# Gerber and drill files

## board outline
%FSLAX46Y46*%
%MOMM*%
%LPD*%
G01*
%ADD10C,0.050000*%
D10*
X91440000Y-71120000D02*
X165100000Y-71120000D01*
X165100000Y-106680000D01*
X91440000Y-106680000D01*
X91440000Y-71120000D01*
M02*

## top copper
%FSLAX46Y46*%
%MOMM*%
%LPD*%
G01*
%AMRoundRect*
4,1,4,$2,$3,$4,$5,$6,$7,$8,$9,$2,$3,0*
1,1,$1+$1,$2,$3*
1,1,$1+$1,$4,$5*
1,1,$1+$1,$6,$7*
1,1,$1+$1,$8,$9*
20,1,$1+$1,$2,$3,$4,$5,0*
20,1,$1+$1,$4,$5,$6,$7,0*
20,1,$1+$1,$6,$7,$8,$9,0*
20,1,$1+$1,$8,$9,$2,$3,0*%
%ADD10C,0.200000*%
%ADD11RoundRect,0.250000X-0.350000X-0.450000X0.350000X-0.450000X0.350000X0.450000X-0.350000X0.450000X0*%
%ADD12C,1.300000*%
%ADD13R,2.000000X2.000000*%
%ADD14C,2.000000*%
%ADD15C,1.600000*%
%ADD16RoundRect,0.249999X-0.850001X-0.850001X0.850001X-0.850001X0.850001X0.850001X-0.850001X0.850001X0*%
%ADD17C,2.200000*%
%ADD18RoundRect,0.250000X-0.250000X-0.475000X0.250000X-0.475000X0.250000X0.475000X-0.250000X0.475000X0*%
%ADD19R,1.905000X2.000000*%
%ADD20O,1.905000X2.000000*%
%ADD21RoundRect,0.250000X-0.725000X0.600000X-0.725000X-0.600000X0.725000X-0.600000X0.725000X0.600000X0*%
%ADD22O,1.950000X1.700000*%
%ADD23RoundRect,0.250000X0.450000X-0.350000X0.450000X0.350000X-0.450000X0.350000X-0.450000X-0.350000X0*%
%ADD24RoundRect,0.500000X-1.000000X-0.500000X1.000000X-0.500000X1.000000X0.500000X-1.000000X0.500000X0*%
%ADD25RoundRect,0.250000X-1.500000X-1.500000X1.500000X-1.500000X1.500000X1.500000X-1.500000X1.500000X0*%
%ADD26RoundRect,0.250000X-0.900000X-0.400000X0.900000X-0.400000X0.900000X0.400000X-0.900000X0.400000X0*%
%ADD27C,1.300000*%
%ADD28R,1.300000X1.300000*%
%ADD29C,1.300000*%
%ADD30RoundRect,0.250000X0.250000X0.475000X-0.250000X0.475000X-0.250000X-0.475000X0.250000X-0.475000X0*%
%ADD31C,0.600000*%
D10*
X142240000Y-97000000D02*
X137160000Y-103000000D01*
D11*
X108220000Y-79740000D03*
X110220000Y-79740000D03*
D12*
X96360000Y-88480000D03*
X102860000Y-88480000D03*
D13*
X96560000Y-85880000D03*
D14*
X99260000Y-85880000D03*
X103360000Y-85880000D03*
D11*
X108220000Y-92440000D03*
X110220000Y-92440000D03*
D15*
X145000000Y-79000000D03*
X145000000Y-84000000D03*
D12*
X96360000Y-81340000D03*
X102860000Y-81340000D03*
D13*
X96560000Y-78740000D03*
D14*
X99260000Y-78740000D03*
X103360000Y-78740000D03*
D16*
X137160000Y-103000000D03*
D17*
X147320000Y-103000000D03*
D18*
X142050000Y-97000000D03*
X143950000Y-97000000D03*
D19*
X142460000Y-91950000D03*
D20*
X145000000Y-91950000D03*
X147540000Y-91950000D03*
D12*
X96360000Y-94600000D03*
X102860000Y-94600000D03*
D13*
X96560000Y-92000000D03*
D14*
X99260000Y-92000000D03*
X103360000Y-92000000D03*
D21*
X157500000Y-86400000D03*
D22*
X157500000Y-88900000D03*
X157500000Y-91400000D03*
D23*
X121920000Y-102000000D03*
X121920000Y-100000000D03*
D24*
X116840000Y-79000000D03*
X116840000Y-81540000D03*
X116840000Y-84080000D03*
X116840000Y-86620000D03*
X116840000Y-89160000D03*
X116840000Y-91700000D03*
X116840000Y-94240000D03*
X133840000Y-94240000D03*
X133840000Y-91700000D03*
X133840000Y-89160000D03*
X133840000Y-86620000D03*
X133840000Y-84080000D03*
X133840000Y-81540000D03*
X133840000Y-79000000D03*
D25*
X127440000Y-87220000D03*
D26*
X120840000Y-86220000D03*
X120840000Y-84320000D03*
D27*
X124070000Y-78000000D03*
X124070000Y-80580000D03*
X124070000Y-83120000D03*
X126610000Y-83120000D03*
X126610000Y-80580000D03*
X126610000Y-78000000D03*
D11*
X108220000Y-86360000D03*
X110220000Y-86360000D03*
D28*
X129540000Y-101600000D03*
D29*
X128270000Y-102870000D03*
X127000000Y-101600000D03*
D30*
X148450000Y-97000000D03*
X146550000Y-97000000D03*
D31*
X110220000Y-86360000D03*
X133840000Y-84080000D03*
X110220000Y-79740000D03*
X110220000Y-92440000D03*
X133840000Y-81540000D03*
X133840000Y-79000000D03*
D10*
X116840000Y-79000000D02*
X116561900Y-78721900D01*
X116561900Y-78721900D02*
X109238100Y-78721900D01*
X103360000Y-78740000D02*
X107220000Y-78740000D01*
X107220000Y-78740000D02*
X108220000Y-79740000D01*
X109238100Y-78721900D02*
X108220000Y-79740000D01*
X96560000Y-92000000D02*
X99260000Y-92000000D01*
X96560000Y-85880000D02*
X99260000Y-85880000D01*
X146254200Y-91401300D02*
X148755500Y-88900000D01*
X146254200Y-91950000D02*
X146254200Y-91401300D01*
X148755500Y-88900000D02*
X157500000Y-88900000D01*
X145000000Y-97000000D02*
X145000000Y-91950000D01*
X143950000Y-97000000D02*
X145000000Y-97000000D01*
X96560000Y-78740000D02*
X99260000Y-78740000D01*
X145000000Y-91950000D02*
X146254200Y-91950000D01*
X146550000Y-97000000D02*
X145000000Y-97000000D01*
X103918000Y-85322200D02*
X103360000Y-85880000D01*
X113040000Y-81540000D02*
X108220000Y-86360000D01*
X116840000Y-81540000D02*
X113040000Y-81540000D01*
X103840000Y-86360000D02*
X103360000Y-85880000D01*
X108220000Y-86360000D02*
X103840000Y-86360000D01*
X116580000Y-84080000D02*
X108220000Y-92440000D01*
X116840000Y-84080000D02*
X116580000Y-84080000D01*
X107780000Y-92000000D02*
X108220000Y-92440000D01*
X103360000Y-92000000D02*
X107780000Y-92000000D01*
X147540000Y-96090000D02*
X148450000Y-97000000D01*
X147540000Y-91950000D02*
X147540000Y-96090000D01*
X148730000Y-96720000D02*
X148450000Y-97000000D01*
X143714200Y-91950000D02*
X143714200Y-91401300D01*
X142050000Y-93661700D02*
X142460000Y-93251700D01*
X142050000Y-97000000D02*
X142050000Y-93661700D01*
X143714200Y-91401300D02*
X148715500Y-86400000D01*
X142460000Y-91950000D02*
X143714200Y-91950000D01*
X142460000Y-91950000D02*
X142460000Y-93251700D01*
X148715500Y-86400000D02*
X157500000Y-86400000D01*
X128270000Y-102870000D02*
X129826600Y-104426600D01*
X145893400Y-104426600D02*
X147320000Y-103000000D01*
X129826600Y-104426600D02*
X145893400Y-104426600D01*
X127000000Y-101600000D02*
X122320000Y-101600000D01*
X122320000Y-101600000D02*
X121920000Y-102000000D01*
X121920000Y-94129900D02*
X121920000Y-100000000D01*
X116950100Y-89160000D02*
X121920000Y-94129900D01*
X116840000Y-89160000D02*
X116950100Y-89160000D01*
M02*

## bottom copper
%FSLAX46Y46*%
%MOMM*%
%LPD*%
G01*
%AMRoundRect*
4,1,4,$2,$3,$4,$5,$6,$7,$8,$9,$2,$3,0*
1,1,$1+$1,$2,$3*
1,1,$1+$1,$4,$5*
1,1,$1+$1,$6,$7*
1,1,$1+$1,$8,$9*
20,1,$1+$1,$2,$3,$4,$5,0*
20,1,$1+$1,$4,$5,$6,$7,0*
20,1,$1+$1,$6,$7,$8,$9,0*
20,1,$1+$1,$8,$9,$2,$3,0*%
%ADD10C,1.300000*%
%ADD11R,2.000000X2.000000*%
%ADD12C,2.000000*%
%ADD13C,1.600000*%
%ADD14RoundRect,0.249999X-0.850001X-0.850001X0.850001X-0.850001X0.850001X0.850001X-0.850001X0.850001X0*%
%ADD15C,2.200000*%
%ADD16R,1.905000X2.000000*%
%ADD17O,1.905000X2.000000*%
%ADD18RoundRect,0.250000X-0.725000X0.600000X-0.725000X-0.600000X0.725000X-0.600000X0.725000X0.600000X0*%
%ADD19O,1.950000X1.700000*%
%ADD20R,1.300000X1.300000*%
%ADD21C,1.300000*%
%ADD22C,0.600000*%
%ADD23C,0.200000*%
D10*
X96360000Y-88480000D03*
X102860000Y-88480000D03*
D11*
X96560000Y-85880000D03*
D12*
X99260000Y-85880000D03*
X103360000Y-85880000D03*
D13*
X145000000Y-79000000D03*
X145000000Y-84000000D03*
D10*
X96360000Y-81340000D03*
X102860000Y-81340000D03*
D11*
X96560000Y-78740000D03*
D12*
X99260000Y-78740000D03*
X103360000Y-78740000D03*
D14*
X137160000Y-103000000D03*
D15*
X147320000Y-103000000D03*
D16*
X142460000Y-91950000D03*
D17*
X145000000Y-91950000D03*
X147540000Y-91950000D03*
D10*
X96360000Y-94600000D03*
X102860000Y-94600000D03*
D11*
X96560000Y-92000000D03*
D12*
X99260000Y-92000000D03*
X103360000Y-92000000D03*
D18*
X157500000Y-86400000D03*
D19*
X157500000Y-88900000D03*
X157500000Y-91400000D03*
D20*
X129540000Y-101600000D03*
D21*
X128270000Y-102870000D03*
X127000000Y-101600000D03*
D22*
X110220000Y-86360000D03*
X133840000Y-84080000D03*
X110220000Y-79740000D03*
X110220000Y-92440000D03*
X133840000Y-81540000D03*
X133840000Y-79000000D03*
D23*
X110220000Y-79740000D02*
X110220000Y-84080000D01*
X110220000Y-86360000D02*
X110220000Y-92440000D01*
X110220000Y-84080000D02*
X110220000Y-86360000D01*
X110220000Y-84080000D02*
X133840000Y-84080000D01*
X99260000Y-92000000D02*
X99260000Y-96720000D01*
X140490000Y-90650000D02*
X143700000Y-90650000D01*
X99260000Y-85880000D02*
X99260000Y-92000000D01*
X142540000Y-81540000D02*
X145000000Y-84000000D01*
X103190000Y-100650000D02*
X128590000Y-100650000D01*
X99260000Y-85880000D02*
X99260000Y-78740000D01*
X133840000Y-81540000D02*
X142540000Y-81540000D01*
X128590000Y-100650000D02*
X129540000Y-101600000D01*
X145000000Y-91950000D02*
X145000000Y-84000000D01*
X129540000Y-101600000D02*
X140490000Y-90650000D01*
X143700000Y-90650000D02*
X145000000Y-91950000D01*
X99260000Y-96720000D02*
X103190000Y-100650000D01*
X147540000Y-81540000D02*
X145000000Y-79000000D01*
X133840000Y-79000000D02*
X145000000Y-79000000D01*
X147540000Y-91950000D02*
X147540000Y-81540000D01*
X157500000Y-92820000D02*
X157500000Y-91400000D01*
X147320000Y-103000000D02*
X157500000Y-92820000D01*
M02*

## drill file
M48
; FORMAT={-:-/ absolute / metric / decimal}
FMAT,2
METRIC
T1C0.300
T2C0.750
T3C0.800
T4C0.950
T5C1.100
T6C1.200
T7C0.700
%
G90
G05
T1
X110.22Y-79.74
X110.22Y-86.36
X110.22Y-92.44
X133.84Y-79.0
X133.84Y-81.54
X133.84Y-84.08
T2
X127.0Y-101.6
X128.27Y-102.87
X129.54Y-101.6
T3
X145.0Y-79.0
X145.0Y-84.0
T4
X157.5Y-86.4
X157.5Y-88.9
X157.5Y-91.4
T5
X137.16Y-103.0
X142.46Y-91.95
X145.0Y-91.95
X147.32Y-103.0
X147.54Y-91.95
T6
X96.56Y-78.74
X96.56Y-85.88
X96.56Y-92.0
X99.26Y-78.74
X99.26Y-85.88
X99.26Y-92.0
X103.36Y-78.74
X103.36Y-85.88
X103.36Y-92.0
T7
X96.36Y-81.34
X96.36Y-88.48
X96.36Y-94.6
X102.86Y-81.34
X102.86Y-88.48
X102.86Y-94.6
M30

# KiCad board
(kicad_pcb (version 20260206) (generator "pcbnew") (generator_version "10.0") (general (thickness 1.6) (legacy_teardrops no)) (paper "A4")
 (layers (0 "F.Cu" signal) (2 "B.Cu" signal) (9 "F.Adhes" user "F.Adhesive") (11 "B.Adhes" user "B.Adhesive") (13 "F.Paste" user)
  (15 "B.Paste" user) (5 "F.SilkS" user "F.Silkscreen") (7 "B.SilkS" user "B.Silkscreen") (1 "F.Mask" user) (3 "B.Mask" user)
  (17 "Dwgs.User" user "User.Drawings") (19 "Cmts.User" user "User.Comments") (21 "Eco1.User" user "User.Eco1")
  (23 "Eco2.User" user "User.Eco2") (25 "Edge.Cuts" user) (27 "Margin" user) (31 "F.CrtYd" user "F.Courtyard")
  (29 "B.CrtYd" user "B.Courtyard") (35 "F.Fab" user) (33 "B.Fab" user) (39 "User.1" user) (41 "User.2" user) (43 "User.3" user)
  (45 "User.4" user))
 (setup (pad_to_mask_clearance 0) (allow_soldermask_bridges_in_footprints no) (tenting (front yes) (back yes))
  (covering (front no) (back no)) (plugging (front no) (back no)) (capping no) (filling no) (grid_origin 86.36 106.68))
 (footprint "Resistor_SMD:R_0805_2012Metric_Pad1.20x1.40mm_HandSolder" (layer "F.Cu") (at 109.22 79.74)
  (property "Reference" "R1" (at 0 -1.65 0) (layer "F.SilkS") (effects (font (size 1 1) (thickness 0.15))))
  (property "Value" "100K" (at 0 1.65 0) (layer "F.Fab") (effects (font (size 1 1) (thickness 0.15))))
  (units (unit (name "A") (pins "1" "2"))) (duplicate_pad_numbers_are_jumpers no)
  (pad "1" smd roundrect (at -1 0) (size 1.2 1.4) (layers "F.Cu" "F.Mask" "F.Paste") (roundrect_rratio 0.208333)
   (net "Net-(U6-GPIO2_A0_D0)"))
  (pad "2" smd roundrect (at 1 0) (size 1.2 1.4) (layers "F.Cu" "F.Mask" "F.Paste") (roundrect_rratio 0.208333) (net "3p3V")))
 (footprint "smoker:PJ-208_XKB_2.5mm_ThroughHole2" (layer "F.Cu") (at 94.86 85.88)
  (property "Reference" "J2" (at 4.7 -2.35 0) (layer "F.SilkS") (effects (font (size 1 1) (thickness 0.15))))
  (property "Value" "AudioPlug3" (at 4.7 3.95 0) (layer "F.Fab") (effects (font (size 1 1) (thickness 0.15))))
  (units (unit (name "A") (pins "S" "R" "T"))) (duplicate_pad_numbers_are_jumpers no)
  (pad "" np_thru_hole circle (at 1.5 2.6) (size 1.3 1.3) (drill 0.7) (layers "*.Cu" "*.Mask"))
  (pad "" np_thru_hole circle (at 8 2.6) (size 1.3 1.3) (drill 0.7) (layers "*.Cu" "*.Mask"))
  (pad "R" thru_hole rect (at 1.7 0) (size 2 2) (drill 1.2) (layers "*.Cu" "*.Mask") (remove_unused_layers no) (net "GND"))
  (pad "S" thru_hole circle (at 4.4 0) (size 2 2) (drill 1.2) (layers "*.Cu" "*.Mask") (remove_unused_layers no) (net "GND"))
  (pad "T" thru_hole circle (at 8.5 0) (size 2 2) (drill 1.2) (layers "*.Cu" "*.Mask") (remove_unused_layers no)
   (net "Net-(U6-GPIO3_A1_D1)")))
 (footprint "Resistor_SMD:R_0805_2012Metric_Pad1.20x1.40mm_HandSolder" (layer "F.Cu") (at 109.22 92.44)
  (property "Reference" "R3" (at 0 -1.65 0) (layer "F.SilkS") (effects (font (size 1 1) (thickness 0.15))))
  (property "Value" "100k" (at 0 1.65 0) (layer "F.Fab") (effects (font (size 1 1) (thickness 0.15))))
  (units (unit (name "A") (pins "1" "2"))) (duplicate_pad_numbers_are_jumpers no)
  (pad "1" smd roundrect (at -1 0) (size 1.2 1.4) (layers "F.Cu" "F.Mask" "F.Paste") (roundrect_rratio 0.208333)
   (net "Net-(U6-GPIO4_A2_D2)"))
  (pad "2" smd roundrect (at 1 0) (size 1.2 1.4) (layers "F.Cu" "F.Mask" "F.Paste") (roundrect_rratio 0.208333) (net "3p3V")))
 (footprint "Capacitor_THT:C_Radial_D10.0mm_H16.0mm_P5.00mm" (layer "F.Cu") (at 145 79 -90)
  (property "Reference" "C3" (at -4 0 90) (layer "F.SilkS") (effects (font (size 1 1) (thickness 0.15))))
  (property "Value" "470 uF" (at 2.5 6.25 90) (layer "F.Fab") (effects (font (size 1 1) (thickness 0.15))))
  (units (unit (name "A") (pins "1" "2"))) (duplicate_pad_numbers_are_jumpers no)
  (pad "1" thru_hole circle (at 0 0 270) (size 1.6 1.6) (drill 0.8) (layers "*.Cu" "*.Mask") (remove_unused_layers no) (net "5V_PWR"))
  (pad "2" thru_hole circle (at 5 0 270) (size 1.6 1.6) (drill 0.8) (layers "*.Cu" "*.Mask") (remove_unused_layers no) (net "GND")))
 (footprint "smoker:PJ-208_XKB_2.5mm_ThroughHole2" (layer "F.Cu") (at 94.86 78.74)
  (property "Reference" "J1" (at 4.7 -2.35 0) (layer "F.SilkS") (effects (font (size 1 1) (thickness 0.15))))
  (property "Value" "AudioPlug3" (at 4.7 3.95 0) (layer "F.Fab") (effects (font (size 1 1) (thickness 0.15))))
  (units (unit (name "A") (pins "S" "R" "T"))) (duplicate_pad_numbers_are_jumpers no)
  (pad "" np_thru_hole circle (at 1.5 2.6) (size 1.3 1.3) (drill 0.7) (layers "*.Cu" "*.Mask"))
  (pad "" np_thru_hole circle (at 8 2.6) (size 1.3 1.3) (drill 0.7) (layers "*.Cu" "*.Mask"))
  (pad "R" thru_hole rect (at 1.7 0) (size 2 2) (drill 1.2) (layers "*.Cu" "*.Mask") (remove_unused_layers no) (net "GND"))
  (pad "S" thru_hole circle (at 4.4 0) (size 2 2) (drill 1.2) (layers "*.Cu" "*.Mask") (remove_unused_layers no) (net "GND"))
  (pad "T" thru_hole circle (at 8.5 0) (size 2 2) (drill 1.2) (layers "*.Cu" "*.Mask") (remove_unused_layers no)
   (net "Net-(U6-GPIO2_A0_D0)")))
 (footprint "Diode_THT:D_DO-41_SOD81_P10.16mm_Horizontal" (layer "F.Cu") (at 137.16 103)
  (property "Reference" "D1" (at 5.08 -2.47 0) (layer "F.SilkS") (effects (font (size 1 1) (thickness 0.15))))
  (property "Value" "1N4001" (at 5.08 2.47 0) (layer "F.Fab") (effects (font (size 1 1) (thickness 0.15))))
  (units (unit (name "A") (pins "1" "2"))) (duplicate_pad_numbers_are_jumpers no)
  (pad "1" thru_hole roundrect (at 0 0) (size 2.2 2.2) (drill 1.1) (layers "*.Cu" "*.Mask") (remove_unused_layers no)
   (roundrect_rratio 0.113636) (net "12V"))
  (pad "2" thru_hole circle (at 10.16 0) (size 2.2 2.2) (drill 1.1) (layers "*.Cu" "*.Mask") (remove_unused_layers no) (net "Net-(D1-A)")))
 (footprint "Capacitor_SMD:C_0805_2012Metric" (layer "F.Cu") (at 143 97)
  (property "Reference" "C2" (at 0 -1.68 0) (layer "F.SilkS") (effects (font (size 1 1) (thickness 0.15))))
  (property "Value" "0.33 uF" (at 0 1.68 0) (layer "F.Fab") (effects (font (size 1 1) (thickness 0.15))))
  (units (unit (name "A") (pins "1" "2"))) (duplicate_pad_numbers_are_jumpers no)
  (pad "1" smd roundrect (at -0.95 0) (size 1 1.45) (layers "F.Cu" "F.Mask" "F.Paste") (roundrect_rratio 0.25) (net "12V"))
  (pad "2" smd roundrect (at 0.95 0) (size 1 1.45) (layers "F.Cu" "F.Mask" "F.Paste") (roundrect_rratio 0.25) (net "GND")))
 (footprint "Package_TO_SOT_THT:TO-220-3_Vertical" (layer "F.Cu") (at 142.46 91.95)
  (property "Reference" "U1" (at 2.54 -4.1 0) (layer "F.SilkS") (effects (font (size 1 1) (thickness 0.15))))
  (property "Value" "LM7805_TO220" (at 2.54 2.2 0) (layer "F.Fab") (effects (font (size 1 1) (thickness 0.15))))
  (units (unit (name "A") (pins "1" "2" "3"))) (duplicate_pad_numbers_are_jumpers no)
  (pad "1" thru_hole rect (at 0 0) (size 1.905 2) (drill 1.1) (layers "*.Cu" "*.Mask") (remove_unused_layers no) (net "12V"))
  (pad "2" thru_hole oval (at 2.54 0) (size 1.905 2) (drill 1.1) (layers "*.Cu" "*.Mask") (remove_unused_layers no) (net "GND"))
  (pad "3" thru_hole oval (at 5.08 0) (size 1.905 2) (drill 1.1) (layers "*.Cu" "*.Mask") (remove_unused_layers no) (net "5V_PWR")))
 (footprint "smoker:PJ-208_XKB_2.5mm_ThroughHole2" (layer "F.Cu") (at 94.86 92)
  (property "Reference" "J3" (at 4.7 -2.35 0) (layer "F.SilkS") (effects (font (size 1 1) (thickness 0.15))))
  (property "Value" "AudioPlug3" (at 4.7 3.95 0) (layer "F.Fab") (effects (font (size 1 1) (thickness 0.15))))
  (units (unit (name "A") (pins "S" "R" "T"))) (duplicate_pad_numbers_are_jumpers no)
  (pad "" np_thru_hole circle (at 1.5 2.6) (size 1.3 1.3) (drill 0.7) (layers "*.Cu" "*.Mask"))
  (pad "" np_thru_hole circle (at 8 2.6) (size 1.3 1.3) (drill 0.7) (layers "*.Cu" "*.Mask"))
  (pad "R" thru_hole rect (at 1.7 0) (size 2 2) (drill 1.2) (layers "*.Cu" "*.Mask") (remove_unused_layers no) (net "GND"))
  (pad "S" thru_hole circle (at 4.4 0) (size 2 2) (drill 1.2) (layers "*.Cu" "*.Mask") (remove_unused_layers no) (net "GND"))
  (pad "T" thru_hole circle (at 8.5 0) (size 2 2) (drill 1.2) (layers "*.Cu" "*.Mask") (remove_unused_layers no)
   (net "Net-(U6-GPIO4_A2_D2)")))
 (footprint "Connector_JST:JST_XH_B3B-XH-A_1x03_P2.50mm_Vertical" (layer "F.Cu") (at 157.5 86.4 -90)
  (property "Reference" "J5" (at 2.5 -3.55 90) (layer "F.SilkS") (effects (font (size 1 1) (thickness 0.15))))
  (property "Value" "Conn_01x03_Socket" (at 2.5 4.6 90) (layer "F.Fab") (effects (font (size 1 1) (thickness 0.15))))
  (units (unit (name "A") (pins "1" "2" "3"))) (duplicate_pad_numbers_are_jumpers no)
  (pad "1" thru_hole roundrect (at 0 0 270) (size 1.7 1.95) (drill 0.95) (layers "*.Cu" "*.Mask") (remove_unused_layers no)
   (roundrect_rratio 0.147059) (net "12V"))
  (pad "2" thru_hole oval (at 2.5 0 270) (size 1.7 1.95) (drill 0.95) (layers "*.Cu" "*.Mask") (remove_unused_layers no) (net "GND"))
  (pad "3" thru_hole oval (at 5 0 270) (size 1.7 1.95) (drill 0.95) (layers "*.Cu" "*.Mask") (remove_unused_layers no) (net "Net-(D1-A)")))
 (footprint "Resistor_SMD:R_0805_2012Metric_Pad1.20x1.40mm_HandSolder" (layer "F.Cu") (at 121.92 101 90)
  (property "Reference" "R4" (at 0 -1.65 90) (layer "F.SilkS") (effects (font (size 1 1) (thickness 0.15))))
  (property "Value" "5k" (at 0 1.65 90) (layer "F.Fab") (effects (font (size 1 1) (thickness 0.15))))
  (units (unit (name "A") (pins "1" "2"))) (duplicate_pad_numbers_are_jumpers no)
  (pad "1" smd roundrect (at -1 0 90) (size 1.2 1.4) (layers "F.Cu" "F.Mask" "F.Paste") (roundrect_rratio 0.208333) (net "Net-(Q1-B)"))
  (pad "2" smd roundrect (at 1 0 90) (size 1.2 1.4) (layers "F.Cu" "F.Mask" "F.Paste") (roundrect_rratio 0.208333)
   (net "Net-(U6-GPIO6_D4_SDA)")))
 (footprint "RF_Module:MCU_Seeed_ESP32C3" (layer "F.Cu") (at 125.34 86.62)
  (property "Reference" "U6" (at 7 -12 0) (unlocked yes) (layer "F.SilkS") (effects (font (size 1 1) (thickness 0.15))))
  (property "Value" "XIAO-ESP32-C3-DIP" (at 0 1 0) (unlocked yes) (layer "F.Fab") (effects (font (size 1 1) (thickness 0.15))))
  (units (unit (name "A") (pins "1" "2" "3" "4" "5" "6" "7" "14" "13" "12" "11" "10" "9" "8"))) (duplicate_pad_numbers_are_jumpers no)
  (pad "" smd roundrect (at 1.1 -0.4) (size 1.5 1.5) (layers "F.Paste") (roundrect_rratio 0.1666666667))
  (pad "" smd roundrect (at 1.1 1.6) (size 1.5 1.5) (layers "F.Paste") (roundrect_rratio 0.1666666667))
  (pad "" smd roundrect (at 3.1 -0.4) (size 1.5 1.5) (layers "F.Paste") (roundrect_rratio 0.1666666667))
  (pad "" smd roundrect (at 3.1 1.6) (size 1.5 1.5) (layers "F.Paste") (roundrect_rratio 0.1666666667))
  (pad "1" smd roundrect (at -8.5 -7.62) (size 3 2) (layers "F.Cu" "F.Mask" "F.Paste") (roundrect_rratio 0.25) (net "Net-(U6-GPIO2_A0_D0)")
   (thermal_bridge_angle 45))
  (pad "2" smd roundrect (at -8.5 -5.08) (size 3 2) (layers "F.Cu" "F.Mask" "F.Paste") (roundrect_rratio 0.25) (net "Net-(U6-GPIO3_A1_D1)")
   (thermal_bridge_angle 45))
  (pad "3" smd roundrect (at -8.5 -2.54) (size 3 2) (layers "F.Cu" "F.Mask" "F.Paste") (roundrect_rratio 0.25) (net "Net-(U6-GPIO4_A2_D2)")
   (thermal_bridge_angle 45))
  (pad "4" smd roundrect (at -8.5 0) (size 3 2) (layers "F.Cu" "F.Mask" "F.Paste") (roundrect_rratio 0.25)
   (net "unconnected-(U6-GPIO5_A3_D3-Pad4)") (thermal_bridge_angle 45))
  (pad "5" smd roundrect (at -8.5 2.54) (size 3 2) (layers "F.Cu" "F.Mask" "F.Paste") (roundrect_rratio 0.25) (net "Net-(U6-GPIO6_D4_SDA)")
   (thermal_bridge_angle 45))
  (pad "6" smd roundrect (at -8.5 5.08) (size 3 2) (layers "F.Cu" "F.Mask" "F.Paste") (roundrect_rratio 0.25)
   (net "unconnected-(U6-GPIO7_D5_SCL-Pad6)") (thermal_bridge_angle 45))
  (pad "7" smd roundrect (at -8.5 7.62) (size 3 2) (layers "F.Cu" "F.Mask" "F.Paste") (roundrect_rratio 0.25)
   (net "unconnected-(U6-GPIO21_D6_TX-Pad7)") (thermal_bridge_angle 45))
  (pad "8" smd roundrect (at 8.5 7.62) (size 3 2) (layers "F.Cu" "F.Mask" "F.Paste") (roundrect_rratio 0.25)
   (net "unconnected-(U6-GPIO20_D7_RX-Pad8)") (thermal_bridge_angle 45))
  (pad "9" smd roundrect (at 8.5 5.08) (size 3 2) (layers "F.Cu" "F.Mask" "F.Paste") (roundrect_rratio 0.25)
   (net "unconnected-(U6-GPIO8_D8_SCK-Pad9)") (thermal_bridge_angle 45))
  (pad "10" smd roundrect (at 8.5 2.54) (size 3 2) (layers "F.Cu" "F.Mask" "F.Paste") (roundrect_rratio 0.25)
   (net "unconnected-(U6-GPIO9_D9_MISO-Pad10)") (thermal_bridge_angle 45))
  (pad "11" smd roundrect (at 8.5 0) (size 3 2) (layers "F.Cu" "F.Mask" "F.Paste") (roundrect_rratio 0.25)
   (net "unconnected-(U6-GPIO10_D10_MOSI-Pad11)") (thermal_bridge_angle 45))
  (pad "12" smd roundrect (at 8.5 -2.54) (size 3 2) (layers "F.Cu" "F.Mask" "F.Paste") (roundrect_rratio 0.25) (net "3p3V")
   (thermal_bridge_angle 45))
  (pad "13" smd roundrect (at 8.5 -5.08) (size 3 2) (layers "F.Cu" "F.Mask" "F.Paste") (roundrect_rratio 0.25) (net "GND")
   (thermal_bridge_angle 45))
  (pad "14" smd roundrect (at 8.5 -7.62) (size 3 2) (layers "F.Cu" "F.Mask" "F.Paste") (roundrect_rratio 0.25) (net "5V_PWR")
   (thermal_bridge_angle 45))
  (pad "15" smd roundrect (at 2.1 0.6) (size 3.5 3.5) (layers "F.Cu" "F.Mask") (roundrect_rratio 0.07142857143))
  (pad "16" smd roundrect (at -4.5 -0.4) (size 2.3 1.3) (layers "F.Cu" "F.Mask" "F.Paste") (roundrect_rratio 0.1923076923))
  (pad "17" smd roundrect (at -4.5 -2.3) (size 2.3 1.3) (layers "F.Cu" "F.Mask" "F.Paste") (roundrect_rratio 0.1923076923))
  (pad "18" smd circle (at -1.27 -8.62) (size 1.3 1.3) (layers "F.Cu" "F.Mask" "F.Paste"))
  (pad "19" smd circle (at -1.27 -6.04) (size 1.3 1.3) (layers "F.Cu" "F.Mask" "F.Paste"))
  (pad "20" smd circle (at -1.27 -3.5) (size 1.3 1.3) (layers "F.Cu" "F.Mask" "F.Paste"))
  (pad "21" smd circle (at 1.27 -3.5) (size 1.3 1.3) (layers "F.Cu" "F.Mask" "F.Paste"))
  (pad "22" smd circle (at 1.27 -6.04) (size 1.3 1.3) (layers "F.Cu" "F.Mask" "F.Paste"))
  (pad "23" smd circle (at 1.27 -8.62) (size 1.3 1.3) (layers "F.Cu" "F.Mask" "F.Paste")))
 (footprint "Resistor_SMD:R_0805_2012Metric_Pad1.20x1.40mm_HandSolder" (layer "F.Cu") (at 109.22 86.36)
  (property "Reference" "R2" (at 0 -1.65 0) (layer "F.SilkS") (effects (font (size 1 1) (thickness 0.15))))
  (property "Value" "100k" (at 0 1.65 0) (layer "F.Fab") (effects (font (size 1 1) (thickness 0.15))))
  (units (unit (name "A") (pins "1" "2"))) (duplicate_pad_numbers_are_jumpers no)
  (pad "1" smd roundrect (at -1 0) (size 1.2 1.4) (layers "F.Cu" "F.Mask" "F.Paste") (roundrect_rratio 0.208333)
   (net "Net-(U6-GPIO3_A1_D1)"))
  (pad "2" smd roundrect (at 1 0) (size 1.2 1.4) (layers "F.Cu" "F.Mask" "F.Paste") (roundrect_rratio 0.208333) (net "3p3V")))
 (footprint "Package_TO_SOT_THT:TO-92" (layer "F.Cu") (at 129.54 101.6 180)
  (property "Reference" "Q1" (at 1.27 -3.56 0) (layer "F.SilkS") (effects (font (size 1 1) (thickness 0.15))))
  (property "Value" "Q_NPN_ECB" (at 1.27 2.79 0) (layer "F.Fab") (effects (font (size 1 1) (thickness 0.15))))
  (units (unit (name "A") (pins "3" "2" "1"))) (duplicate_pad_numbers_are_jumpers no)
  (pad "1" thru_hole rect (at 0 0 180) (size 1.3 1.3) (drill 0.75) (layers "*.Cu" "*.Mask") (remove_unused_layers no) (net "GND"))
  (pad "2" thru_hole circle (at 1.27 -1.27 180) (size 1.3 1.3) (drill 0.75) (layers "*.Cu" "*.Mask") (remove_unused_layers no)
   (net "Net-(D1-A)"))
  (pad "3" thru_hole circle (at 2.54 0 180) (size 1.3 1.3) (drill 0.75) (layers "*.Cu" "*.Mask") (remove_unused_layers no)
   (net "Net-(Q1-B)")))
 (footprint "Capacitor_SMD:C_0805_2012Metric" (layer "F.Cu") (at 147.5 97 180)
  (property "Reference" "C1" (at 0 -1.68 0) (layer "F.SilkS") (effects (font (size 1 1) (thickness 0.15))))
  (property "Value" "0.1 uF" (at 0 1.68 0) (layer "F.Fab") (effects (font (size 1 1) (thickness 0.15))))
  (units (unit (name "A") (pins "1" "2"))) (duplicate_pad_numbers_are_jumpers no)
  (pad "1" smd roundrect (at -0.95 0 180) (size 1 1.45) (layers "F.Cu" "F.Mask" "F.Paste") (roundrect_rratio 0.25) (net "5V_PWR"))
  (pad "2" smd roundrect (at 0.95 0 180) (size 1 1.45) (layers "F.Cu" "F.Mask" "F.Paste") (roundrect_rratio 0.25) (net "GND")))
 (gr_line (start 142.24 97) (end 137.16 103) (stroke (width 0.2) (type default)) (layer "F.Cu") (net "12V"))
 (gr_rect (start 91.44 71.12) (end 165.1 106.68) (stroke (width 0.05) (type default)) (fill no) (layer "Edge.Cuts"))
 (segment (start 116.84 79) (end 116.5619 78.7219) (width 0.2) (layer "F.Cu") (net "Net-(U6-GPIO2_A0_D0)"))
 (segment (start 116.5619 78.7219) (end 109.2381 78.7219) (width 0.2) (layer "F.Cu") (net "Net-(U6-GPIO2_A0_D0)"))
 (segment (start 103.36 78.74) (end 107.22 78.74) (width 0.2) (layer "F.Cu") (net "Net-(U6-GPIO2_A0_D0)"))
 (segment (start 107.22 78.74) (end 108.22 79.74) (width 0.2) (layer "F.Cu") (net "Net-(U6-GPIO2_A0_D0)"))
 (segment (start 109.2381 78.7219) (end 108.22 79.74) (width 0.2) (layer "F.Cu") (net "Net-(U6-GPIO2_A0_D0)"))
 (via (at 110.22 86.36) (size 0.6) (drill 0.3) (layers "F.Cu" "B.Cu") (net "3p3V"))
 (via (at 133.84 84.08) (size 0.6) (drill 0.3) (layers "F.Cu" "B.Cu") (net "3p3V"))
 (via (at 110.22 79.74) (size 0.6) (drill 0.3) (layers "F.Cu" "B.Cu") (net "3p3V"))
 (via (at 110.22 92.44) (size 0.6) (drill 0.3) (layers "F.Cu" "B.Cu") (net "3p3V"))
 (segment (start 110.22 79.74) (end 110.22 84.08) (width 0.2) (layer "B.Cu") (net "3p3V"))
 (segment (start 110.22 86.36) (end 110.22 92.44) (width 0.2) (layer "B.Cu") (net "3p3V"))
 (segment (start 110.22 84.08) (end 110.22 86.36) (width 0.2) (layer "B.Cu") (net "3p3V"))
 (segment (start 110.22 84.08) (end 133.84 84.08) (width 0.2) (layer "B.Cu") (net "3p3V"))
 (segment (start 96.56 92) (end 99.26 92) (width 0.2) (layer "F.Cu") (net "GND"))
 (segment (start 96.56 85.88) (end 99.26 85.88) (width 0.2) (layer "F.Cu") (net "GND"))
 (segment (start 146.2542 91.4013) (end 148.7555 88.9) (width 0.2) (layer "F.Cu") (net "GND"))
 (segment (start 146.2542 91.95) (end 146.2542 91.4013) (width 0.2) (layer "F.Cu") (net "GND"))
 (segment (start 148.7555 88.9) (end 157.5 88.9) (width 0.2) (layer "F.Cu") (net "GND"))
 (segment (start 145 97) (end 145 91.95) (width 0.2) (layer "F.Cu") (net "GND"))
 (segment (start 143.95 97) (end 145 97) (width 0.2) (layer "F.Cu") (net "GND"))
 (segment (start 96.56 78.74) (end 99.26 78.74) (width 0.2) (layer "F.Cu") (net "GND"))
 (segment (start 145 91.95) (end 146.2542 91.95) (width 0.2) (layer "F.Cu") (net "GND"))
 (segment (start 146.55 97) (end 145 97) (width 0.2) (layer "F.Cu") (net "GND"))
 (via (at 133.84 81.54) (size 0.6) (drill 0.3) (layers "F.Cu" "B.Cu") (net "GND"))
 (segment (start 99.26 92) (end 99.26 96.72) (width 0.2) (layer "B.Cu") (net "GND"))
 (segment (start 140.49 90.65) (end 143.7 90.65) (width 0.2) (layer "B.Cu") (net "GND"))
 (segment (start 99.26 85.88) (end 99.26 92) (width 0.2) (layer "B.Cu") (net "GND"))
 (segment (start 142.54 81.54) (end 145 84) (width 0.2) (layer "B.Cu") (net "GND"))
 (segment (start 103.19 100.65) (end 128.59 100.65) (width 0.2) (layer "B.Cu") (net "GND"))
 (segment (start 99.26 85.88) (end 99.26 78.74) (width 0.2) (layer "B.Cu") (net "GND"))
 (segment (start 133.84 81.54) (end 142.54 81.54) (width 0.2) (layer "B.Cu") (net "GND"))
 (segment (start 128.59 100.65) (end 129.54 101.6) (width 0.2) (layer "B.Cu") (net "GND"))
 (segment (start 145 91.95) (end 145 84) (width 0.2) (layer "B.Cu") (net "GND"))
 (segment (start 129.54 101.6) (end 140.49 90.65) (width 0.2) (layer "B.Cu") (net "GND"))
 (segment (start 143.7 90.65) (end 145 91.95) (width 0.2) (layer "B.Cu") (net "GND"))
 (segment (start 99.26 96.72) (end 103.19 100.65) (width 0.2) (layer "B.Cu") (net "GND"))
 (segment (start 103.918 85.3222) (end 103.36 85.88) (width 0.2) (layer "F.Cu") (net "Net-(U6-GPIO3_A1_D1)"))
 (segment (start 113.04 81.54) (end 108.22 86.36) (width 0.2) (layer "F.Cu") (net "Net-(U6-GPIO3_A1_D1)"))
 (segment (start 116.84 81.54) (end 113.04 81.54) (width 0.2) (layer "F.Cu") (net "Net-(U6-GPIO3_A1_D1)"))
 (segment (start 103.84 86.36) (end 103.36 85.88) (width 0.2) (layer "F.Cu") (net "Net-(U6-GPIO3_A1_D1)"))
 (segment (start 108.22 86.36) (end 103.84 86.36) (width 0.2) (layer "F.Cu") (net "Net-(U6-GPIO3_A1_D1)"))
 (segment (start 116.58 84.08) (end 108.22 92.44) (width 0.2) (layer "F.Cu") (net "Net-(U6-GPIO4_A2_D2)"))
 (segment (start 116.84 84.08) (end 116.58 84.08) (width 0.2) (layer "F.Cu") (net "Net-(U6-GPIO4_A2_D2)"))
 (segment (start 107.78 92) (end 108.22 92.44) (width 0.2) (layer "F.Cu") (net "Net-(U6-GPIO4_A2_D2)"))
 (segment (start 103.36 92) (end 107.78 92) (width 0.2) (layer "F.Cu") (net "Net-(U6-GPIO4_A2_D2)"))
 (segment (start 147.54 96.09) (end 148.45 97) (width 0.2) (layer "F.Cu") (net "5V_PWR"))
 (segment (start 147.54 91.95) (end 147.54 96.09) (width 0.2) (layer "F.Cu") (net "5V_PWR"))
 (segment (start 148.73 96.72) (end 148.45 97) (width 0.2) (layer "F.Cu") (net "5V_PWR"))
 (via (at 133.84 79) (size 0.6) (drill 0.3) (layers "F.Cu" "B.Cu") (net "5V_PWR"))
 (segment (start 147.54 81.54) (end 145 79) (width 0.2) (layer "B.Cu") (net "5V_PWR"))
 (segment (start 133.84 79) (end 145 79) (width 0.2) (layer "B.Cu") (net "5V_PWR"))
 (segment (start 147.54 91.95) (end 147.54 81.54) (width 0.2) (layer "B.Cu") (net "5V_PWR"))
 (segment (start 143.7142 91.95) (end 143.7142 91.4013) (width 0.2) (layer "F.Cu") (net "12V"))
 (segment (start 142.05 93.6617) (end 142.46 93.2517) (width 0.2) (layer "F.Cu") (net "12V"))
 (segment (start 142.05 97) (end 142.05 93.6617) (width 0.2) (layer "F.Cu") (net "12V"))
 (segment (start 143.7142 91.4013) (end 148.7155 86.4) (width 0.2) (layer "F.Cu") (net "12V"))
 (segment (start 142.46 91.95) (end 143.7142 91.95) (width 0.2) (layer "F.Cu") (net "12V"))
 (segment (start 142.46 91.95) (end 142.46 93.2517) (width 0.2) (layer "F.Cu") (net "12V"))
 (segment (start 148.7155 86.4) (end 157.5 86.4) (width 0.2) (layer "F.Cu") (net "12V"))
 (segment (start 128.27 102.87) (end 129.8266 104.4266) (width 0.2) (layer "F.Cu") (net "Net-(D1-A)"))
 (segment (start 145.8934 104.4266) (end 147.32 103) (width 0.2) (layer "F.Cu") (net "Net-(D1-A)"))
 (segment (start 129.8266 104.4266) (end 145.8934 104.4266) (width 0.2) (layer "F.Cu") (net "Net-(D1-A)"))
 (segment (start 157.5 92.82) (end 157.5 91.4) (width 0.2) (layer "B.Cu") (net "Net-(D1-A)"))
 (segment (start 147.32 103) (end 157.5 92.82) (width 0.2) (layer "B.Cu") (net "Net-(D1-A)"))
 (segment (start 127 101.6) (end 122.32 101.6) (width 0.2) (layer "F.Cu") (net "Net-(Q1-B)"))
 (segment (start 122.32 101.6) (end 121.92 102) (width 0.2) (layer "F.Cu") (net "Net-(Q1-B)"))
 (segment (start 121.92 94.1299) (end 121.92 100) (width 0.2) (layer "F.Cu") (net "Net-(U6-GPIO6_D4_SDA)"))
 (segment (start 116.9501 89.16) (end 121.92 94.1299) (width 0.2) (layer "F.Cu") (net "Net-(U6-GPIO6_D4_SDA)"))
 (segment (start 116.84 89.16) (end 116.9501 89.16) (width 0.2) (layer "F.Cu") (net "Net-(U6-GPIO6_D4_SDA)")))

